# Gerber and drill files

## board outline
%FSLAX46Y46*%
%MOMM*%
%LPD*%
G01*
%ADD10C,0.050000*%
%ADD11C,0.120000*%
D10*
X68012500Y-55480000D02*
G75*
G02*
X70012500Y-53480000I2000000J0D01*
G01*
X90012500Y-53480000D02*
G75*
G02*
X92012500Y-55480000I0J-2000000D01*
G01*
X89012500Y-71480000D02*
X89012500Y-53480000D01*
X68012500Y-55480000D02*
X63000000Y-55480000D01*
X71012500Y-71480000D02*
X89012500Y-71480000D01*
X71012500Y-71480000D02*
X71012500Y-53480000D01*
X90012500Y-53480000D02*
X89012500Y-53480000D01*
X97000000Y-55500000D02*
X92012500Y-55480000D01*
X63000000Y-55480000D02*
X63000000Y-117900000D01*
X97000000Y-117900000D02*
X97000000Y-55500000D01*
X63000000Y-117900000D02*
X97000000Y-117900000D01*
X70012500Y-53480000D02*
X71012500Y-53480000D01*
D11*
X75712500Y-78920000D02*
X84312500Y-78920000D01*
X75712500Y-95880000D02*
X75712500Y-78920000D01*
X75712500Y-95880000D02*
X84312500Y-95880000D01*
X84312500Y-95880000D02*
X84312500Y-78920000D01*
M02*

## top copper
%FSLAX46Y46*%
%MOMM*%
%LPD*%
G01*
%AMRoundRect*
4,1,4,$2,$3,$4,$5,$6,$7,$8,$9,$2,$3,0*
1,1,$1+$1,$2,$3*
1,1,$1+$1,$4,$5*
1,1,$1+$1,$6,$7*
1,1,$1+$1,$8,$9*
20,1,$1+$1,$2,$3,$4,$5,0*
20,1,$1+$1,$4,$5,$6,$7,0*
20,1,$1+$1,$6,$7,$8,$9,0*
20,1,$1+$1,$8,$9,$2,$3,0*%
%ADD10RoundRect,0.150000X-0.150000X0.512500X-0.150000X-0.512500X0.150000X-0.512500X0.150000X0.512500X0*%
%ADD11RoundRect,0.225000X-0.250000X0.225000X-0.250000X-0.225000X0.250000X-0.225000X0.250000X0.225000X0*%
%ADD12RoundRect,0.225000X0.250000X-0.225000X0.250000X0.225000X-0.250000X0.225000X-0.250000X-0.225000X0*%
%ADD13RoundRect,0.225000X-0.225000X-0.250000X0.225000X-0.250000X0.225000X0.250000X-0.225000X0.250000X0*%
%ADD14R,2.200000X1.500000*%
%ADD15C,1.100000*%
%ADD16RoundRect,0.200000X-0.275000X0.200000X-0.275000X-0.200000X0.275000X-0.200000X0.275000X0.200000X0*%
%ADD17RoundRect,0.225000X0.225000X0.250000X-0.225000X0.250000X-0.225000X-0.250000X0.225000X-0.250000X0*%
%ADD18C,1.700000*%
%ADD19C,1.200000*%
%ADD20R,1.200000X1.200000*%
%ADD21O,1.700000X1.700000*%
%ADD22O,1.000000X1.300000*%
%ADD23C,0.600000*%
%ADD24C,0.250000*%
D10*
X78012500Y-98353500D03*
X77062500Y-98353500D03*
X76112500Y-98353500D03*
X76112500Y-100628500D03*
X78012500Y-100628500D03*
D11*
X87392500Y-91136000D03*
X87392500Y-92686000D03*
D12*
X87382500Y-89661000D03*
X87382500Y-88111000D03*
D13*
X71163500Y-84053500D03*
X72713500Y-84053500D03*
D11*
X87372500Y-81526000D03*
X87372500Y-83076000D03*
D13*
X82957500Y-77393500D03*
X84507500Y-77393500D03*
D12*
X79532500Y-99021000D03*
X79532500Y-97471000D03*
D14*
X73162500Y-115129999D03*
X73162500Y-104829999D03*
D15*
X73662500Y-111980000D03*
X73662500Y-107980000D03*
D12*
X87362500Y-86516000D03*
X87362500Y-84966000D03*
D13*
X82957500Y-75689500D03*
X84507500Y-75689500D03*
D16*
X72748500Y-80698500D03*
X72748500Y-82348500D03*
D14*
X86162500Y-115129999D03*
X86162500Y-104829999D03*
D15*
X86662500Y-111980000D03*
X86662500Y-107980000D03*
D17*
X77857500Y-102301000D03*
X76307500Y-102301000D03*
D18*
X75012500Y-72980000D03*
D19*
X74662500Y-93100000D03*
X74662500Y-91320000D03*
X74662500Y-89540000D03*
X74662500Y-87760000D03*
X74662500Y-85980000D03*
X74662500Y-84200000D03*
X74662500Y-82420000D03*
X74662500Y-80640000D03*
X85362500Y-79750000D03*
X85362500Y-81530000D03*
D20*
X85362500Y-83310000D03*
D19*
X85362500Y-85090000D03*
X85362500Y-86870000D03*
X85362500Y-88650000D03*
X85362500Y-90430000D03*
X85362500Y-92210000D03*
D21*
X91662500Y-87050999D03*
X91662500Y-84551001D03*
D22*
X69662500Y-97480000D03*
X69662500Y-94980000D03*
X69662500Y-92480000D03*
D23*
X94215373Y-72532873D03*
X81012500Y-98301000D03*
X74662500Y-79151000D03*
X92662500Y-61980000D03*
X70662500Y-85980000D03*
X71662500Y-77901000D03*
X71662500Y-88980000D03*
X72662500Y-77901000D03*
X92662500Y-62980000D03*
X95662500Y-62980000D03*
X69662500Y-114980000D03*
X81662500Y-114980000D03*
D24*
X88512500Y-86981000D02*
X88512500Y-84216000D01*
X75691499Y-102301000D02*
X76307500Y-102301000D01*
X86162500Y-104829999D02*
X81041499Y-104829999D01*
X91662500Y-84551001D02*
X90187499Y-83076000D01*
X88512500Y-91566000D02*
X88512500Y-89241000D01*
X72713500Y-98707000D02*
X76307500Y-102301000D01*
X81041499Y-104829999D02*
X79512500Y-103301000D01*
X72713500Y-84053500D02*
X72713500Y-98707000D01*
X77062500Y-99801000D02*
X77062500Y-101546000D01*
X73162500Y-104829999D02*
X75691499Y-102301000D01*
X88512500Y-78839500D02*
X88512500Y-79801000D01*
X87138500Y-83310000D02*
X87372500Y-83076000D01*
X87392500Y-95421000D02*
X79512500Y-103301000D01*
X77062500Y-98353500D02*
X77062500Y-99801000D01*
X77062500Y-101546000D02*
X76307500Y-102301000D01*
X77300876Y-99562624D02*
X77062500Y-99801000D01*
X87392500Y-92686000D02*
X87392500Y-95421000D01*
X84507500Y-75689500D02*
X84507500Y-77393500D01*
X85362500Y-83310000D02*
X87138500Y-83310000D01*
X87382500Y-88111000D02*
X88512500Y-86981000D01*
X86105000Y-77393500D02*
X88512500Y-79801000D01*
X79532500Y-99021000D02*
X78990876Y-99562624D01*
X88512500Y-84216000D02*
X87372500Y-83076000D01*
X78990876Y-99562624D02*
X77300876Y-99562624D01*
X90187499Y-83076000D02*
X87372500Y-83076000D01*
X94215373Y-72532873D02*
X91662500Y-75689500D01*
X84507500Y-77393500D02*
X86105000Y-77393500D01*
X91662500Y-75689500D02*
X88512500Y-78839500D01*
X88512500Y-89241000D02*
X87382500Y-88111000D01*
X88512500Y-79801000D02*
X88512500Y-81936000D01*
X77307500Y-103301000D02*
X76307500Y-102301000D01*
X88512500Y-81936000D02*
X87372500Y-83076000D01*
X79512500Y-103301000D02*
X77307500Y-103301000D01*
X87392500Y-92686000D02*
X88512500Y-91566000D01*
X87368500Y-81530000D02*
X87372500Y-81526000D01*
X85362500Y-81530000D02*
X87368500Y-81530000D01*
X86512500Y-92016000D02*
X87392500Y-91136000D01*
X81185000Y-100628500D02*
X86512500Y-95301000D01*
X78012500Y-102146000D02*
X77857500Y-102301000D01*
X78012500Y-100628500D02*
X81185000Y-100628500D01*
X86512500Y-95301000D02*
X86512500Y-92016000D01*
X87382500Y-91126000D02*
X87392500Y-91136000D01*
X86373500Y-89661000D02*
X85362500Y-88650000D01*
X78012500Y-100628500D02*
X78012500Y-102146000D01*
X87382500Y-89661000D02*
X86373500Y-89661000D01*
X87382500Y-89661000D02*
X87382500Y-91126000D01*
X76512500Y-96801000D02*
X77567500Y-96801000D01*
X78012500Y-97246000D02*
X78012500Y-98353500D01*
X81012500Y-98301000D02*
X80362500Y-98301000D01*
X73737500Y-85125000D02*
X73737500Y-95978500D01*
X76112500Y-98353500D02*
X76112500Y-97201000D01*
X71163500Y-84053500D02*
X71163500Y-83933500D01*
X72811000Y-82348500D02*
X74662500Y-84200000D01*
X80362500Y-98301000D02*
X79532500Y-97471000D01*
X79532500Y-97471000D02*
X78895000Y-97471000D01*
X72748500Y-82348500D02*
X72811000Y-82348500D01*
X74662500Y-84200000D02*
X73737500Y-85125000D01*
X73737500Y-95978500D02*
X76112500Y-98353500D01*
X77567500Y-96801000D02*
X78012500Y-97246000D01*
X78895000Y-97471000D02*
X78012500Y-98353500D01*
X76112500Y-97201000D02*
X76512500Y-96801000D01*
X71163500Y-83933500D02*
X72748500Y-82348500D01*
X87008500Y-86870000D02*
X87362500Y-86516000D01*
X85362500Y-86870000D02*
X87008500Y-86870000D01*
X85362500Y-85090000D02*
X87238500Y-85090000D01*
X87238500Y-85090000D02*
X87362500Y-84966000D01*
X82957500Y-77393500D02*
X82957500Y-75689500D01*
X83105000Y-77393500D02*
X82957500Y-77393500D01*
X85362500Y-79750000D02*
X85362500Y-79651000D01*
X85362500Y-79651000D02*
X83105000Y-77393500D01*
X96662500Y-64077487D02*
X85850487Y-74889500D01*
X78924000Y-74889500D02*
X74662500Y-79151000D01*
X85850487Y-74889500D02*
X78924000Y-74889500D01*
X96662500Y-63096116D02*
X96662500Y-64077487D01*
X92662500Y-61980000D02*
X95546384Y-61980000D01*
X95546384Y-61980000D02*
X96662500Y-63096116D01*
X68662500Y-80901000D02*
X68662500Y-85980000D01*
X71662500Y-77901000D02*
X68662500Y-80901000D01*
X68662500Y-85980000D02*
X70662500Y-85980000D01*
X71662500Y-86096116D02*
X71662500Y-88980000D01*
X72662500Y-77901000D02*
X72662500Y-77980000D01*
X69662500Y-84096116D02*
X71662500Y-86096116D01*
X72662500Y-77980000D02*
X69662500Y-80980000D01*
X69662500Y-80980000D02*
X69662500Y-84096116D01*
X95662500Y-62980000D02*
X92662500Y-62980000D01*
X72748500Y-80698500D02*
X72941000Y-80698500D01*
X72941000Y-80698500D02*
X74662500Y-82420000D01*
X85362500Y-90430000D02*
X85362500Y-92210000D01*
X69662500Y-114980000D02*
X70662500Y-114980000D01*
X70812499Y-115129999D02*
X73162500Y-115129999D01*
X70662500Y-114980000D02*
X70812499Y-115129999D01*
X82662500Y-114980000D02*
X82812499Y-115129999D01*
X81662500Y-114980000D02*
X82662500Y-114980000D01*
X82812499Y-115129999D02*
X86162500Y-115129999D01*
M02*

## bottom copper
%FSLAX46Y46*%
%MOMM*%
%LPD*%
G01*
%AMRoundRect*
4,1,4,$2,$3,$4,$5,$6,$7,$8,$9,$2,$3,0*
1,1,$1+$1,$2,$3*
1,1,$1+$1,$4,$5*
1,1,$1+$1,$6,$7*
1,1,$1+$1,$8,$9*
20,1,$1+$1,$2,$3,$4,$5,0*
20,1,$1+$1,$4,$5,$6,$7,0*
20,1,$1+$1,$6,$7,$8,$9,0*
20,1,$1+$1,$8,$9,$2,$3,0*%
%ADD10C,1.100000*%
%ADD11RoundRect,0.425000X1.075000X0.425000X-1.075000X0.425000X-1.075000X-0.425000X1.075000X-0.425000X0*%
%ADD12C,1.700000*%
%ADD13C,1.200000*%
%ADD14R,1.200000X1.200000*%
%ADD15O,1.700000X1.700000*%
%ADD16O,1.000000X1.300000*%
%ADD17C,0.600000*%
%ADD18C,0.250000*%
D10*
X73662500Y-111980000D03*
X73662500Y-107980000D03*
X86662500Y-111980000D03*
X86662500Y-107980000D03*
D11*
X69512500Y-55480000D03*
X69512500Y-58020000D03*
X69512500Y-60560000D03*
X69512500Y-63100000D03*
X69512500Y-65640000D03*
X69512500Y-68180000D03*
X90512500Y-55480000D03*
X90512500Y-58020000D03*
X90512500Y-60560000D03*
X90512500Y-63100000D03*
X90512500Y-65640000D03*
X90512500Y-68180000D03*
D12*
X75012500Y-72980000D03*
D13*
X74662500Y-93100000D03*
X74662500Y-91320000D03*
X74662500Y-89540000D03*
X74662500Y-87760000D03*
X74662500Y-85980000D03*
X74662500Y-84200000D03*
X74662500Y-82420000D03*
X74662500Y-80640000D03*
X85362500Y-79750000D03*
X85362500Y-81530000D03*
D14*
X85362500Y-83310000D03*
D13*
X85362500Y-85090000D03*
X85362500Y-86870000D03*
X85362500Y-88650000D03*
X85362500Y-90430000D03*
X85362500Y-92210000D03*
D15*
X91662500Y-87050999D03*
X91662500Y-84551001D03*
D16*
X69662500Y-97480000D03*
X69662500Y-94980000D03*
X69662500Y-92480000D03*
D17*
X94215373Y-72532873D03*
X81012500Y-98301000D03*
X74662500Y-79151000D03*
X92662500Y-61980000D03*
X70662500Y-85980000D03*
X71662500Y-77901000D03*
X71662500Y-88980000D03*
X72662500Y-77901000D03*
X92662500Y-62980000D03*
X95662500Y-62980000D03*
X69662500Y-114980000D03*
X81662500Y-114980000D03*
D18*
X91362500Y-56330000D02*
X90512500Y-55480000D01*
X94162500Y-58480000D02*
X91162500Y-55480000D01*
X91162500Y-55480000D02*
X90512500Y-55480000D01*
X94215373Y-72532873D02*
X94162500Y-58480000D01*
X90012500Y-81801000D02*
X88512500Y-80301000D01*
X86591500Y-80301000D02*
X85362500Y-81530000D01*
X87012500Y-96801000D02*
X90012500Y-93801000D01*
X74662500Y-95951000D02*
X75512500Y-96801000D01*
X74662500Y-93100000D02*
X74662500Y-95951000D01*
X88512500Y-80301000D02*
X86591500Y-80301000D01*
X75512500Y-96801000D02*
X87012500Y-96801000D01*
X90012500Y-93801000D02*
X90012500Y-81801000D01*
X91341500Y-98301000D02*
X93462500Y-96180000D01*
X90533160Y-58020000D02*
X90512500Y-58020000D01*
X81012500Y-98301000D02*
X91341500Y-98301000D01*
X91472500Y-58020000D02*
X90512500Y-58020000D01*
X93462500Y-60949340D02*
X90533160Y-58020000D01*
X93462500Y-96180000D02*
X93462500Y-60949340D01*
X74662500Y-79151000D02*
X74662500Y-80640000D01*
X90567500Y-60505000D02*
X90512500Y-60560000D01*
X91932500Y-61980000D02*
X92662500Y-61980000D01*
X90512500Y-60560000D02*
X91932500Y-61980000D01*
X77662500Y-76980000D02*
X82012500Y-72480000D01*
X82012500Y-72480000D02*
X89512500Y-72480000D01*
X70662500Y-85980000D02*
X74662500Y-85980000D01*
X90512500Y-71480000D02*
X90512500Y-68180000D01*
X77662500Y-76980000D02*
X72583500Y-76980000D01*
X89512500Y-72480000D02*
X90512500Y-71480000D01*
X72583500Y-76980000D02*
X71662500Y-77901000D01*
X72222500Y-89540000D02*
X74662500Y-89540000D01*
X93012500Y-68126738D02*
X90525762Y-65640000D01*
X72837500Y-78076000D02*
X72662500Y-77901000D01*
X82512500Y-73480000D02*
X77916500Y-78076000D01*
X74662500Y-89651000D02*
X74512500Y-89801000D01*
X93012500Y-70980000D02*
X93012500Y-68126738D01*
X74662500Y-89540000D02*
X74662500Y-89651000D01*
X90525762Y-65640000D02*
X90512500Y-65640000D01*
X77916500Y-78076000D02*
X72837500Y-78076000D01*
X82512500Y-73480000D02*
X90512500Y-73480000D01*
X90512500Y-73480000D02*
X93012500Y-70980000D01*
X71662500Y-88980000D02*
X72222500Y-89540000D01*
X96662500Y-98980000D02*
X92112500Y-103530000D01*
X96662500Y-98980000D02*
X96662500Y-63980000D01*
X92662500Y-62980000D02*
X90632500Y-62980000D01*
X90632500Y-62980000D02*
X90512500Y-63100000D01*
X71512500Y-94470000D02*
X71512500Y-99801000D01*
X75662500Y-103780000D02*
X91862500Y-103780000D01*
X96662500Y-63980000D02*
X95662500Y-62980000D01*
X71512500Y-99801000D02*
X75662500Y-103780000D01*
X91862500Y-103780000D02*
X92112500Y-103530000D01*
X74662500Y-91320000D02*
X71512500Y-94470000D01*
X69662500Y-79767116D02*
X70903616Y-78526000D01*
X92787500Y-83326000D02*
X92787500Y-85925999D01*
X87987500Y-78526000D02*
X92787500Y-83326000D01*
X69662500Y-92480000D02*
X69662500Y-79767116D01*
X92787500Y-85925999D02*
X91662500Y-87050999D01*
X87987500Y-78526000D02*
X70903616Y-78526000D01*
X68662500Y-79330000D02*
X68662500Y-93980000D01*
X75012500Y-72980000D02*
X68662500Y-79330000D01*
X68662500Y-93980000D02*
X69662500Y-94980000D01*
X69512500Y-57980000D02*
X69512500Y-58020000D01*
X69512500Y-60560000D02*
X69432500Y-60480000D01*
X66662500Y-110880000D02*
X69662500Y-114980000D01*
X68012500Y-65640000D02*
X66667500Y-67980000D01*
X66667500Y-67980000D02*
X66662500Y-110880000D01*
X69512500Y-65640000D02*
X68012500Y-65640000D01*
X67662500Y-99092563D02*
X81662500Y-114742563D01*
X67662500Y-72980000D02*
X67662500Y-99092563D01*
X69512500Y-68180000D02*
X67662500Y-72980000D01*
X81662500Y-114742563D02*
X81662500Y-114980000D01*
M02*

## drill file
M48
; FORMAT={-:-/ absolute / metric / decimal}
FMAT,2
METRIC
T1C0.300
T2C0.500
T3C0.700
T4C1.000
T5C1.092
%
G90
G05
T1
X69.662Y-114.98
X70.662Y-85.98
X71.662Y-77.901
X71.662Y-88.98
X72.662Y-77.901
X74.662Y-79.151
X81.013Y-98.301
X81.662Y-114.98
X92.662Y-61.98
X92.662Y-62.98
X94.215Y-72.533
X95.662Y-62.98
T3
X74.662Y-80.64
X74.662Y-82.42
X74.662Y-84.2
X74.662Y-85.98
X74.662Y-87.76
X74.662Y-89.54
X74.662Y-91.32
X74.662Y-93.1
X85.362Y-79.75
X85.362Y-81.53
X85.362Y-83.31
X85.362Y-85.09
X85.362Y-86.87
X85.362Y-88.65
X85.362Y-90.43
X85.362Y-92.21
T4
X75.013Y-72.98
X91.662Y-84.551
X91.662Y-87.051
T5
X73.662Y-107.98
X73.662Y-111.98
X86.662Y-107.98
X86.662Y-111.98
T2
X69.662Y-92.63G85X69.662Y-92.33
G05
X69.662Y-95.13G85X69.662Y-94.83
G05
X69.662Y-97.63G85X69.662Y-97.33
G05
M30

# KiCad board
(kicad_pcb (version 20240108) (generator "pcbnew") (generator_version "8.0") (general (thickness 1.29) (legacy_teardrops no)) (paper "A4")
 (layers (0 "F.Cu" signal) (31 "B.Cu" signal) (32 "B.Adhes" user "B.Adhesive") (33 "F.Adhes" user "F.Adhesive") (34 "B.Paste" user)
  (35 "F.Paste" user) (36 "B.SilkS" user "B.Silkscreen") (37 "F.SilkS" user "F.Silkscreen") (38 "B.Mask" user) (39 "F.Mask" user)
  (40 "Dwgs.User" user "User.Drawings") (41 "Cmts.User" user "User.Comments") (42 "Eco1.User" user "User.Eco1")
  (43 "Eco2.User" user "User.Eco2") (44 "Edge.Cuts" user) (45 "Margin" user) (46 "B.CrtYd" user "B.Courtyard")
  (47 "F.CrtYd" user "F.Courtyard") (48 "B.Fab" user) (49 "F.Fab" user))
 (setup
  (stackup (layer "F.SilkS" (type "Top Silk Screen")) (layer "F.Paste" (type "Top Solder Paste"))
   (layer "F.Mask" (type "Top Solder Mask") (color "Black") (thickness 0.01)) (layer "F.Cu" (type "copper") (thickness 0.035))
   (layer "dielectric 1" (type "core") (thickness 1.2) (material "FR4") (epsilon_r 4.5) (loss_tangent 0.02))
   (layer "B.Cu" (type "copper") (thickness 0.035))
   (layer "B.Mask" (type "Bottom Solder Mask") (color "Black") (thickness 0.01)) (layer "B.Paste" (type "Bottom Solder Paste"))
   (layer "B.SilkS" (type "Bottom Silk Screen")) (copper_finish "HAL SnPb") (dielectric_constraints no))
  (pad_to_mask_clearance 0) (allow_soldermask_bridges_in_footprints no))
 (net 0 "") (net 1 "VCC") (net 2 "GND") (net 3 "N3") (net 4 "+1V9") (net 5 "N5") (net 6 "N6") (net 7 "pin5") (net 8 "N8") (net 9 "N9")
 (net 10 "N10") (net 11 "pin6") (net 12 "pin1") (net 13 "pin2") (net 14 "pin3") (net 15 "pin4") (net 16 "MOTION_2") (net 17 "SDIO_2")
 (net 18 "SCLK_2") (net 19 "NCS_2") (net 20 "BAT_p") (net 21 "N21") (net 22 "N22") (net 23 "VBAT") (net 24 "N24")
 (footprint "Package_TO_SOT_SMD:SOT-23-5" (layer "F.Cu") (at 77.0625 99.491 -90)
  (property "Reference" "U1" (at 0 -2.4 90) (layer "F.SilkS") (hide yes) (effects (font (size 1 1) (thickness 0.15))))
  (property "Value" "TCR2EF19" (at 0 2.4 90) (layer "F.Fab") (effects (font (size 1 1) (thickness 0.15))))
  (pad "1" smd roundrect (at -1.1375 -0.95 270) (size 1.325 0.6) (layers "F.Cu" "F.Paste" "F.Mask") (roundrect_rratio 0.25) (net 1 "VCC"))
  (pad "2" smd roundrect (at -1.1375 0 270) (size 1.325 0.6) (layers "F.Cu" "F.Paste" "F.Mask") (roundrect_rratio 0.25) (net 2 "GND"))
  (pad "3" smd roundrect (at -1.1375 0.95 270) (size 1.325 0.6) (layers "F.Cu" "F.Paste" "F.Mask") (roundrect_rratio 0.25) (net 1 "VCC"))
  (pad "4" smd roundrect (at 1.1375 0.95 270) (size 1.325 0.6) (layers "F.Cu" "F.Paste" "F.Mask") (roundrect_rratio 0.25) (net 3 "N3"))
  (pad "5" smd roundrect (at 1.1375 -0.95 270) (size 1.325 0.6) (layers "F.Cu" "F.Paste" "F.Mask") (roundrect_rratio 0.25) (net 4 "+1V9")))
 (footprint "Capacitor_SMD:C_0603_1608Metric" (layer "F.Cu") (at 87.3925 91.911 -90)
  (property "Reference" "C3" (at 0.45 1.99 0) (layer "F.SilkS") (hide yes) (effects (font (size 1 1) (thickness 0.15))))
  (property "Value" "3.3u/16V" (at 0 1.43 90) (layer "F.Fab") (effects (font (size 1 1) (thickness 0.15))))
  (pad "1" smd roundrect (at -0.775 0 270) (size 0.9 0.95) (layers "F.Cu" "F.Paste" "F.Mask") (roundrect_rratio 0.25) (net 4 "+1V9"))
  (pad "2" smd roundrect (at 0.775 0 270) (size 0.9 0.95) (layers "F.Cu" "F.Paste" "F.Mask") (roundrect_rratio 0.25) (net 2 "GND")))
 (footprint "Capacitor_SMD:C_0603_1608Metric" (layer "F.Cu") (at 87.3825 88.886 90)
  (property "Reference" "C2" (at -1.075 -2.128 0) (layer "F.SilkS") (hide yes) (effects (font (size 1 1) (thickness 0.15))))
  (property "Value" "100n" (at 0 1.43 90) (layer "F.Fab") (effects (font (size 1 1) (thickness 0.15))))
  (pad "1" smd roundrect (at -0.775 0 90) (size 0.9 0.95) (layers "F.Cu" "F.Paste" "F.Mask") (roundrect_rratio 0.25) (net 4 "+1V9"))
  (pad "2" smd roundrect (at 0.775 0 90) (size 0.9 0.95) (layers "F.Cu" "F.Paste" "F.Mask") (roundrect_rratio 0.25) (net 2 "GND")))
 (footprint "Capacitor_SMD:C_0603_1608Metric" (layer "F.Cu") (at 71.9385 84.0535)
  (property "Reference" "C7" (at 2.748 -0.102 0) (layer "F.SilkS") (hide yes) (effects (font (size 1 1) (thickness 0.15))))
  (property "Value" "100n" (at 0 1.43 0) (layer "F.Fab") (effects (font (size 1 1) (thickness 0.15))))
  (pad "1" smd roundrect (at -0.775 0) (size 0.9 0.95) (layers "F.Cu" "F.Paste" "F.Mask") (roundrect_rratio 0.25) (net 1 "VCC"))
  (pad "2" smd roundrect (at 0.775 0) (size 0.9 0.95) (layers "F.Cu" "F.Paste" "F.Mask") (roundrect_rratio 0.25) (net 2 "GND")))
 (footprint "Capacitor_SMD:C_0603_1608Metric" (layer "F.Cu") (at 87.3725 82.301 -90)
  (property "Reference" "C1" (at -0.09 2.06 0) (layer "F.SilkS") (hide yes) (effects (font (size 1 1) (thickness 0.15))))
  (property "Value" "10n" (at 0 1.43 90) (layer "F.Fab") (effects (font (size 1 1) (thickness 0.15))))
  (pad "1" smd roundrect (at -0.775 0 270) (size 0.9 0.95) (layers "F.Cu" "F.Paste" "F.Mask") (roundrect_rratio 0.25) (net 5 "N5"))
  (pad "2" smd roundrect (at 0.775 0 270) (size 0.9 0.95) (layers "F.Cu" "F.Paste" "F.Mask") (roundrect_rratio 0.25) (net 2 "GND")))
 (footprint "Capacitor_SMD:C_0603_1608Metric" (layer "F.Cu") (at 83.7325 77.3935)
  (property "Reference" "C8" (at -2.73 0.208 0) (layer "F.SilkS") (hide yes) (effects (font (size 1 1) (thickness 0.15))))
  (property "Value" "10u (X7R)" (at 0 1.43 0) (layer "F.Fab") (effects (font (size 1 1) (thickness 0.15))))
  (pad "1" smd roundrect (at -0.775 0) (size 0.9 0.95) (layers "F.Cu" "F.Paste" "F.Mask") (roundrect_rratio 0.25) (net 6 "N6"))
  (pad "2" smd roundrect (at 0.775 0) (size 0.9 0.95) (layers "F.Cu" "F.Paste" "F.Mask") (roundrect_rratio 0.25) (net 2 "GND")))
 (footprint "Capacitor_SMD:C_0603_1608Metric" (layer "F.Cu") (at 79.5325 98.246 90)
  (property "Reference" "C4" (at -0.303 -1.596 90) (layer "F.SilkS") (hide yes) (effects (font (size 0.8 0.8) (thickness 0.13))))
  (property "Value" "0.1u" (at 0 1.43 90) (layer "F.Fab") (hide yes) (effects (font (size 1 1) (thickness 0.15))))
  (pad "1" smd roundrect (at -0.775 0 90) (size 0.9 0.95) (layers "F.Cu" "F.Paste" "F.Mask") (roundrect_rratio 0.25) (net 2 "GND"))
  (pad "2" smd roundrect (at 0.775 0 90) (size 0.9 0.95) (layers "F.Cu" "F.Paste" "F.Mask") (roundrect_rratio 0.25) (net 1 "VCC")))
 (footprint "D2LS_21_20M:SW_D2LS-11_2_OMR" (layer "F.Cu") (at 73.6625 109.98 90)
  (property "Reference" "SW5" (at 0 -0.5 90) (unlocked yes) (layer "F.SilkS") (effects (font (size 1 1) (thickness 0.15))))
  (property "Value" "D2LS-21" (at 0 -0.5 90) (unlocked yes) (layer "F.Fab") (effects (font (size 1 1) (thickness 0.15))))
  (pad "1" smd rect (at -5.149999 -0.5 90) (size 1.5 2.2) (layers "F.Cu" "F.Paste" "F.Mask") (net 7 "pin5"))
  (pad "2" smd rect (at 5.150001 -0.5 90) (size 1.5 2.2) (layers "F.Cu" "F.Paste" "F.Mask") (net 2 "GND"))
  (pad "3" thru_hole circle (at -2 0 90) (size 1.1 1.1) (drill 1.0922) (layers "*.Cu" "*.Mask") (remove_unused_layers no))
  (pad "4" thru_hole circle (at 2 0 90) (size 1.1 1.1) (drill 1.0922) (layers "*.Cu" "*.Mask") (remove_unused_layers no)))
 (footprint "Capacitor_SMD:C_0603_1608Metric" (layer "F.Cu") (at 87.3625 85.741 90)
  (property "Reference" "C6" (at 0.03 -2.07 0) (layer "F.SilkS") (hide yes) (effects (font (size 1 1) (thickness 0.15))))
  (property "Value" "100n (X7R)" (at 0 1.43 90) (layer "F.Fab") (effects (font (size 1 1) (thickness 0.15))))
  (pad "1" smd roundrect (at -0.775 0 90) (size 0.9 0.95) (layers "F.Cu" "F.Paste" "F.Mask") (roundrect_rratio 0.25) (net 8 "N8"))
  (pad "2" smd roundrect (at 0.775 0 90) (size 0.9 0.95) (layers "F.Cu" "F.Paste" "F.Mask") (roundrect_rratio 0.25) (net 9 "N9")))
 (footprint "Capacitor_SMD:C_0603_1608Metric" (layer "F.Cu") (at 83.7325 75.6895)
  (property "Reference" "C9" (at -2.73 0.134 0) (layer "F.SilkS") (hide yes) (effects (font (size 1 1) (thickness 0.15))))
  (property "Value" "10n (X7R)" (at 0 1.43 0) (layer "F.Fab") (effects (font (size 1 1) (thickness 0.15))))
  (pad "1" smd roundrect (at -0.775 0) (size 0.9 0.95) (layers "F.Cu" "F.Paste" "F.Mask") (roundrect_rratio 0.25) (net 6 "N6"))
  (pad "2" smd roundrect (at 0.775 0) (size 0.9 0.95) (layers "F.Cu" "F.Paste" "F.Mask") (roundrect_rratio 0.25) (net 2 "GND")))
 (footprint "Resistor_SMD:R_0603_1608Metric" (layer "F.Cu") (at 72.7485 81.5235 -90)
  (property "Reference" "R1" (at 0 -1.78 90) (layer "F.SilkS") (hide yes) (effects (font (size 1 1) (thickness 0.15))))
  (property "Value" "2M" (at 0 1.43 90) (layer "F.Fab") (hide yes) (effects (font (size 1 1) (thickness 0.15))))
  (pad "1" smd roundrect (at -0.825 0 270) (size 0.8 0.95) (layers "F.Cu" "F.Paste" "F.Mask") (roundrect_rratio 0.25) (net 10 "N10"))
  (pad "2" smd roundrect (at 0.825 0 270) (size 0.8 0.95) (layers "F.Cu" "F.Paste" "F.Mask") (roundrect_rratio 0.25) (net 1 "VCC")))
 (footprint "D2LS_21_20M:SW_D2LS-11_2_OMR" (layer "F.Cu") (at 86.6625 109.98 90)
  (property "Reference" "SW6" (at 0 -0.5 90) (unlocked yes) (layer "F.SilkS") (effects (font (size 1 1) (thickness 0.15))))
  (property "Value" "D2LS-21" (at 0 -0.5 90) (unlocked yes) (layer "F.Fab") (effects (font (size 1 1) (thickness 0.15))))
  (pad "1" smd rect (at -5.149999 -0.5 90) (size 1.5 2.2) (layers "F.Cu" "F.Paste" "F.Mask") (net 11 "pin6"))
  (pad "2" smd rect (at 5.150001 -0.5 90) (size 1.5 2.2) (layers "F.Cu" "F.Paste" "F.Mask") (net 2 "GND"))
  (pad "3" thru_hole circle (at -2 0 90) (size 1.1 1.1) (drill 1.0922) (layers "*.Cu" "*.Mask") (remove_unused_layers no))
  (pad "4" thru_hole circle (at 2 0 90) (size 1.1 1.1) (drill 1.0922) (layers "*.Cu" "*.Mask") (remove_unused_layers no)))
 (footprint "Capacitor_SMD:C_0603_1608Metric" (layer "F.Cu") (at 77.0825 102.301 180)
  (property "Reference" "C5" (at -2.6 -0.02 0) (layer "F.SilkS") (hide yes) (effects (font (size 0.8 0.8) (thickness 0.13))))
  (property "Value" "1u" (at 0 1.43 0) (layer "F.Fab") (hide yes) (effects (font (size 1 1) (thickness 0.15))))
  (pad "1" smd roundrect (at -0.775 0 180) (size 0.9 0.95) (layers "F.Cu" "F.Paste" "F.Mask") (roundrect_rratio 0.25) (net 4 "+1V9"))
  (pad "2" smd roundrect (at 0.775 0 180) (size 0.9 0.95) (layers "F.Cu" "F.Paste" "F.Mask") (roundrect_rratio 0.25) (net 2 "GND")))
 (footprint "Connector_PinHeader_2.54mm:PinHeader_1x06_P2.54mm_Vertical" (layer "B.Cu") (at 69.5125 55.48 180)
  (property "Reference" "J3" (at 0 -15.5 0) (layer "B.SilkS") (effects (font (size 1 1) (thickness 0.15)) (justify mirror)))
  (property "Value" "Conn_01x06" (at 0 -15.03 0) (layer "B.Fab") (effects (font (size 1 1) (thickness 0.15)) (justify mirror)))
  (pad "1" smd roundrect (at 0 0 180) (size 3 1.7) (layers "B.Cu" "B.Paste" "B.Mask") (roundrect_rratio 0.25) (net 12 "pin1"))
  (pad "2" smd roundrect (at 0 -2.54 180) (size 3 1.7) (layers "B.Cu" "B.Paste" "B.Mask") (roundrect_rratio 0.25) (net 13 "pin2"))
  (pad "3" smd roundrect (at 0 -5.08 180) (size 3 1.7) (layers "B.Cu" "B.Paste" "B.Mask") (roundrect_rratio 0.25) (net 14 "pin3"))
  (pad "4" smd roundrect (at 0 -7.62 180) (size 3 1.7) (layers "B.Cu" "B.Paste" "B.Mask") (roundrect_rratio 0.25) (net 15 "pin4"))
  (pad "5" smd roundrect (at 0 -10.16 180) (size 3 1.7) (layers "B.Cu" "B.Paste" "B.Mask") (roundrect_rratio 0.25) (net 7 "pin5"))
  (pad "6" smd roundrect (at 0 -12.7 180) (size 3 1.7) (layers "B.Cu" "B.Paste" "B.Mask") (roundrect_rratio 0.25) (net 11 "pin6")))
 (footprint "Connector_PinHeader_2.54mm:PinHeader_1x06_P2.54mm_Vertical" (layer "B.Cu") (at 90.5125 55.48 180)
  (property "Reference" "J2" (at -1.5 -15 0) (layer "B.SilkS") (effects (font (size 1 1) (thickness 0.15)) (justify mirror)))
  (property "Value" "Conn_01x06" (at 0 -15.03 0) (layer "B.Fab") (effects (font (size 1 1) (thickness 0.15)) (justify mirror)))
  (pad "1" smd roundrect (at 0 0 180) (size 3 1.7) (layers "B.Cu" "B.Paste" "B.Mask") (roundrect_rratio 0.25) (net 2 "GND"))
  (pad "2" smd roundrect (at 0 -2.54 180) (size 3 1.7) (layers "B.Cu" "B.Paste" "B.Mask") (roundrect_rratio 0.25) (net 1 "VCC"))
  (pad "3" smd roundrect (at 0 -5.08 180) (size 3 1.7) (layers "B.Cu" "B.Paste" "B.Mask") (roundrect_rratio 0.25) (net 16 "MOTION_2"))
  (pad "4" smd roundrect (at 0 -7.62 180) (size 3 1.7) (layers "B.Cu" "B.Paste" "B.Mask") (roundrect_rratio 0.25) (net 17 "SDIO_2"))
  (pad "5" smd roundrect (at 0 -10.16 180) (size 3 1.7) (layers "B.Cu" "B.Paste" "B.Mask") (roundrect_rratio 0.25) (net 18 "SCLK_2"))
  (pad "6" smd roundrect (at 0 -12.7 180) (size 3 1.7) (layers "B.Cu" "B.Paste" "B.Mask") (roundrect_rratio 0.25) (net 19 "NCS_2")))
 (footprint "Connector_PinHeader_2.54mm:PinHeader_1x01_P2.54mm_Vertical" (layer "B.Cu") (at 75.0125 72.98 180)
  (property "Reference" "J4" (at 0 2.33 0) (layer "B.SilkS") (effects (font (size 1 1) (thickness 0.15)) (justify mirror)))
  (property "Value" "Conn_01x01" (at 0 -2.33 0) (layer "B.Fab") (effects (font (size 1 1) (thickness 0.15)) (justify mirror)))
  (pad "1" thru_hole circle (at 0 0 180) (size 1.7 1.7) (drill 1) (layers "*.Cu" "*.Mask") (remove_unused_layers no) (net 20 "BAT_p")))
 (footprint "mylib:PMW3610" (layer "B.Cu") (at 74.6625 93.1)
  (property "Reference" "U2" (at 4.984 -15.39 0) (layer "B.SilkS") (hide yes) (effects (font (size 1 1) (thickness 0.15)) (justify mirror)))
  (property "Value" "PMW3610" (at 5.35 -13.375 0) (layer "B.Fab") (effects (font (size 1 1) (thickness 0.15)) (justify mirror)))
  (fp_line (start 1.05 -14.18) (end 9.65 -14.18) (stroke (width 0.12) (type solid)) (layer "Edge.Cuts"))
  (fp_line (start 1.05 2.78) (end 1.05 -14.18) (stroke (width 0.12) (type solid)) (layer "Edge.Cuts"))
  (fp_line (start 1.05 2.78) (end 9.65 2.78) (stroke (width 0.12) (type solid)) (layer "Edge.Cuts"))
  (fp_line (start 9.65 2.78) (end 9.65 -14.18) (stroke (width 0.12) (type solid)) (layer "Edge.Cuts"))
  (pad "1" thru_hole circle (at 0 0) (size 1.2 1.2) (drill 0.7) (layers "*.Cu" "*.Mask") (remove_unused_layers no) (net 5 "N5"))
  (pad "2" thru_hole circle (at 0 -1.78) (size 1.2 1.2) (drill 0.7) (layers "*.Cu" "*.Mask") (remove_unused_layers no) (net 17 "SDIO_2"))
  (pad "3" thru_hole circle (at 0 -3.56) (size 1.2 1.2) (drill 0.7) (layers "*.Cu" "*.Mask") (remove_unused_layers no) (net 18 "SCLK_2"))
  (pad "4" thru_hole circle (at 0 -5.34) (size 1.2 1.2) (drill 0.7) (layers "*.Cu" "*.Mask") (remove_unused_layers no) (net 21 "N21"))
  (pad "5" thru_hole circle (at 0 -7.12) (size 1.2 1.2) (drill 0.7) (layers "*.Cu" "*.Mask") (remove_unused_layers no) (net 19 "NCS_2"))
  (pad "6" thru_hole circle (at 0 -8.9) (size 1.2 1.2) (drill 0.7) (layers "*.Cu" "*.Mask") (remove_unused_layers no) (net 1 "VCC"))
  (pad "7" thru_hole circle (at 0 -10.68) (size 1.2 1.2) (drill 0.7) (layers "*.Cu" "*.Mask") (remove_unused_layers no) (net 10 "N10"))
  (pad "8" thru_hole circle (at 0 -12.46) (size 1.2 1.2) (drill 0.7) (layers "*.Cu" "*.Mask") (remove_unused_layers no) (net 16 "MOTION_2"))
  (pad "9" thru_hole circle (at 10.7 -13.35) (size 1.2 1.2) (drill 0.7) (layers "*.Cu" "*.Mask") (remove_unused_layers no) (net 6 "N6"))
  (pad "10" thru_hole circle (at 10.7 -11.57) (size 1.2 1.2) (drill 0.7) (layers "*.Cu" "*.Mask") (remove_unused_layers no) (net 5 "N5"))
  (pad "11" thru_hole rect (at 10.7 -9.79) (size 1.2 1.2) (drill 0.7) (layers "*.Cu" "*.Mask") (remove_unused_layers no) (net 2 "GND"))
  (pad "12" thru_hole circle (at 10.7 -8.01) (size 1.2 1.2) (drill 0.7) (layers "*.Cu" "*.Mask") (remove_unused_layers no) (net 9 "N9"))
  (pad "13" thru_hole circle (at 10.7 -6.23) (size 1.2 1.2) (drill 0.7) (layers "*.Cu" "*.Mask") (remove_unused_layers no) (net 8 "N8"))
  (pad "14" thru_hole circle (at 10.7 -4.45) (size 1.2 1.2) (drill 0.7) (layers "*.Cu" "*.Mask") (remove_unused_layers no) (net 4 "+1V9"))
  (pad "15" thru_hole circle (at 10.7 -2.67) (size 1.2 1.2) (drill 0.7) (layers "*.Cu" "*.Mask") (remove_unused_layers no) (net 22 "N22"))
  (pad "16" thru_hole circle (at 10.7 -0.89) (size 1.2 1.2) (drill 0.7) (layers "*.Cu" "*.Mask") (remove_unused_layers no) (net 22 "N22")))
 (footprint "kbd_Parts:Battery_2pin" (layer "B.Cu") (at 91.6625 85.801 90)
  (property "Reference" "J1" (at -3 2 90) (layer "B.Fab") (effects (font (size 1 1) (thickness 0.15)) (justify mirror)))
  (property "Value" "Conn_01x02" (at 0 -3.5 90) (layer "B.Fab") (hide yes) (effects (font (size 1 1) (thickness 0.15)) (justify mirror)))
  (pad "1" thru_hole oval (at -1.249999 0 90) (size 1.7 1.7) (drill oval 1) (layers "*.Cu" "*.Mask") (remove_unused_layers no)
   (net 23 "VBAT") (clearance 0.15))
  (pad "2" thru_hole oval (at 1.249999 0 90) (size 1.7 1.7) (drill oval 1) (layers "*.Cu" "*.Mask") (remove_unused_layers no) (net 2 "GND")
   (clearance 0.15)))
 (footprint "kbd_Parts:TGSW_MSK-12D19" (layer "B.Cu") (at 70.7125 94.98 90)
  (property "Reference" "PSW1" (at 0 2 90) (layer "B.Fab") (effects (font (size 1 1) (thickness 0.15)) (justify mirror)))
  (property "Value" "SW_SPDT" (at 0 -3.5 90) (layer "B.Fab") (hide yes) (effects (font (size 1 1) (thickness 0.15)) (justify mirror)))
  (pad "1" thru_hole oval (at -2.5 -1.05 90) (size 1.3 1) (drill oval 0.8 0.5) (layers "*.Cu" "*.Mask") (remove_unused_layers no)
   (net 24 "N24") (clearance 0.15))
  (pad "2" thru_hole oval (at 0 -1.05 90) (size 1.3 1) (drill oval 0.8 0.5) (layers "*.Cu" "*.Mask") (remove_unused_layers no)
   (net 20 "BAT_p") (clearance 0.15))
  (pad "3" thru_hole oval (at 2.5 -1.05 90) (size 1.3 1) (drill oval 0.8 0.5) (layers "*.Cu" "*.Mask") (remove_unused_layers no)
   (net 23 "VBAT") (clearance 0.15)))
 (gr_arc (start 68.0125 55.48) (mid 68.598286 54.065786) (end 70.0125 53.48) (stroke (width 0.05) (type default)) (layer "Edge.Cuts"))
 (gr_arc (start 90.0125 53.48) (mid 91.426714 54.065786) (end 92.0125 55.48) (stroke (width 0.05) (type default)) (layer "Edge.Cuts"))
 (gr_line (start 89.0125 71.48) (end 89.0125 53.48) (stroke (width 0.05) (type default)) (layer "Edge.Cuts"))
 (gr_line (start 68.0125 55.48) (end 63 55.48) (stroke (width 0.05) (type default)) (layer "Edge.Cuts"))
 (gr_line (start 71.0125 71.48) (end 89.0125 71.48) (stroke (width 0.05) (type default)) (layer "Edge.Cuts"))
 (gr_line (start 71.0125 71.48) (end 71.0125 53.48) (stroke (width 0.05) (type default)) (layer "Edge.Cuts"))
 (gr_line (start 90.0125 53.48) (end 89.0125 53.48) (stroke (width 0.05) (type default)) (layer "Edge.Cuts"))
 (gr_line (start 97 55.5) (end 92.0125 55.48) (stroke (width 0.05) (type default)) (layer "Edge.Cuts"))
 (gr_line (start 63 55.48) (end 63 117.9) (stroke (width 0.05) (type default)) (layer "Edge.Cuts"))
 (gr_line (start 97 117.9) (end 97 55.5) (stroke (width 0.05) (type default)) (layer "Edge.Cuts"))
 (gr_line (start 63 117.9) (end 97 117.9) (stroke (width 0.05) (type default)) (layer "Edge.Cuts"))
 (gr_line (start 70.0125 53.48) (end 71.0125 53.48) (stroke (width 0.05) (type default)) (layer "Edge.Cuts"))
 (segment (start 88.5125 86.981) (end 88.5125 84.216) (width 0.25) (layer "F.Cu") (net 2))
 (segment (start 75.691499 102.301) (end 76.3075 102.301) (width 0.25) (layer "F.Cu") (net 2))
 (segment (start 86.1625 104.829999) (end 81.041499 104.829999) (width 0.25) (layer "F.Cu") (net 2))
 (segment (start 91.6625 84.551001) (end 90.187499 83.076) (width 0.25) (layer "F.Cu") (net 2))
 (segment (start 88.5125 91.566) (end 88.5125 89.241) (width 0.25) (layer "F.Cu") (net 2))
 (segment (start 72.7135 98.707) (end 76.3075 102.301) (width 0.25) (layer "F.Cu") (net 2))
 (segment (start 81.041499 104.829999) (end 79.5125 103.301) (width 0.25) (layer "F.Cu") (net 2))
 (segment (start 72.7135 84.0535) (end 72.7135 98.707) (width 0.25) (layer "F.Cu") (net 2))
 (segment (start 77.0625 99.801) (end 77.0625 101.546) (width 0.25) (layer "F.Cu") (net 2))
 (segment (start 73.1625 104.829999) (end 75.691499 102.301) (width 0.25) (layer "F.Cu") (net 2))
 (segment (start 88.5125 78.8395) (end 88.5125 79.801) (width 0.25) (layer "F.Cu") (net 2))
 (segment (start 87.1385 83.31) (end 87.3725 83.076) (width 0.25) (layer "F.Cu") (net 2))
 (segment (start 87.3925 95.421) (end 79.5125 103.301) (width 0.25) (layer "F.Cu") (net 2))
 (segment (start 77.0625 98.3535) (end 77.0625 99.801) (width 0.25) (layer "F.Cu") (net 2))
 (segment (start 77.0625 101.546) (end 76.3075 102.301) (width 0.25) (layer "F.Cu") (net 2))
 (segment (start 77.300876 99.562624) (end 77.0625 99.801) (width 0.25) (layer "F.Cu") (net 2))
 (segment (start 87.3925 92.686) (end 87.3925 95.421) (width 0.25) (layer "F.Cu") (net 2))
 (segment (start 84.5075 75.6895) (end 84.5075 77.3935) (width 0.25) (layer "F.Cu") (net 2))
 (segment (start 85.3625 83.31) (end 87.1385 83.31) (width 0.25) (layer "F.Cu") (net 2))
 (segment (start 87.3825 88.111) (end 88.5125 86.981) (width 0.25) (layer "F.Cu") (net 2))
 (segment (start 86.105 77.3935) (end 88.5125 79.801) (width 0.25) (layer "F.Cu") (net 2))
 (segment (start 79.5325 99.021) (end 78.990876 99.562624) (width 0.25) (layer "F.Cu") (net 2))
 (segment (start 88.5125 84.216) (end 87.3725 83.076) (width 0.25) (layer "F.Cu") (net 2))
 (segment (start 78.990876 99.562624) (end 77.300876 99.562624) (width 0.25) (layer "F.Cu") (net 2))
 (segment (start 90.187499 83.076) (end 87.3725 83.076) (width 0.25) (layer "F.Cu") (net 2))
 (segment (start 94.215373 72.532873) (end 91.6625 75.6895) (width 0.25) (layer "F.Cu") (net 2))
 (segment (start 84.5075 77.3935) (end 86.105 77.3935) (width 0.25) (layer "F.Cu") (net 2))
 (segment (start 91.6625 75.6895) (end 88.5125 78.8395) (width 0.25) (layer "F.Cu") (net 2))
 (segment (start 88.5125 89.241) (end 87.3825 88.111) (width 0.25) (layer "F.Cu") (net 2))
 (segment (start 88.5125 79.801) (end 88.5125 81.936) (width 0.25) (layer "F.Cu") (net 2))
 (segment (start 77.3075 103.301) (end 76.3075 102.301) (width 0.25) (layer "F.Cu") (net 2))
 (segment (start 88.5125 81.936) (end 87.3725 83.076) (width 0.25) (layer "F.Cu") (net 2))
 (segment (start 79.5125 103.301) (end 77.3075 103.301) (width 0.25) (layer "F.Cu") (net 2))
 (segment (start 87.3925 92.686) (end 88.5125 91.566) (width 0.25) (layer "F.Cu") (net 2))
 (via (at 94.215373 72.532873) (size 0.6) (drill 0.3) (layers "F.Cu" "B.Cu") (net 2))
 (segment (start 91.3625 56.33) (end 90.5125 55.48) (width 0.25) (layer "B.Cu") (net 2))
 (segment (start 94.1625 58.48) (end 91.1625 55.48) (width 0.25) (layer "B.Cu") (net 2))
 (segment (start 91.1625 55.48) (end 90.5125 55.48) (width 0.25) (layer "B.Cu") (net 2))
 (segment (start 94.215373 72.532873) (end 94.1625 58.48) (width 0.25) (layer "B.Cu") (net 2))
 (segment (start 87.3685 81.53) (end 87.3725 81.526) (width 0.25) (layer "F.Cu") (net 5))
 (segment (start 85.3625 81.53) (end 87.3685 81.53) (width 0.25) (layer "F.Cu") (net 5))
 (segment (start 90.0125 81.801) (end 88.5125 80.301) (width 0.25) (layer "B.Cu") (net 5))
 (segment (start 86.5915 80.301) (end 85.3625 81.53) (width 0.25) (layer "B.Cu") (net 5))
 (segment (start 87.0125 96.801) (end 90.0125 93.801) (width 0.25) (layer "B.Cu") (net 5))
 (segment (start 74.6625 95.951) (end 75.5125 96.801) (width 0.25) (layer "B.Cu") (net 5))
 (segment (start 74.6625 93.1) (end 74.6625 95.951) (width 0.25) (layer "B.Cu") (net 5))
 (segment (start 88.5125 80.301) (end 86.5915 80.301) (width 0.25) (layer "B.Cu") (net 5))
 (segment (start 75.5125 96.801) (end 87.0125 96.801) (width 0.25) (layer "B.Cu") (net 5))
 (segment (start 90.0125 93.801) (end 90.0125 81.801) (width 0.25) (layer "B.Cu") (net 5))
 (segment (start 86.5125 92.016) (end 87.3925 91.136) (width 0.25) (layer "F.Cu") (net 4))
 (segment (start 81.185 100.6285) (end 86.5125 95.301) (width 0.25) (layer "F.Cu") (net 4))
 (segment (start 78.0125 102.146) (end 77.8575 102.301) (width 0.25) (layer "F.Cu") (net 4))
 (segment (start 78.0125 100.6285) (end 81.185 100.6285) (width 0.25) (layer "F.Cu") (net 4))
 (segment (start 86.5125 95.301) (end 86.5125 92.016) (width 0.25) (layer "F.Cu") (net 4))
 (segment (start 87.3825 91.126) (end 87.3925 91.136) (width 0.25) (layer "F.Cu") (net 4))
 (segment (start 86.3735 89.661) (end 85.3625 88.65) (width 0.25) (layer "F.Cu") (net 4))
 (segment (start 78.0125 100.6285) (end 78.0125 102.146) (width 0.25) (layer "F.Cu") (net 4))
 (segment (start 87.3825 89.661) (end 86.3735 89.661) (width 0.25) (layer "F.Cu") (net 4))
 (segment (start 87.3825 89.661) (end 87.3825 91.126) (width 0.25) (layer "F.Cu") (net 4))
 (segment (start 76.5125 96.801) (end 77.5675 96.801) (width 0.25) (layer "F.Cu") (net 1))
 (segment (start 78.0125 97.246) (end 78.0125 98.3535) (width 0.25) (layer "F.Cu") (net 1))
 (segment (start 81.0125 98.301) (end 80.3625 98.301) (width 0.25) (layer "F.Cu") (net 1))
 (segment (start 73.7375 85.125) (end 73.7375 95.9785) (width 0.25) (layer "F.Cu") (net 1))
 (segment (start 76.1125 98.3535) (end 76.1125 97.201) (width 0.25) (layer "F.Cu") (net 1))
 (segment (start 71.1635 84.0535) (end 71.1635 83.9335) (width 0.25) (layer "F.Cu") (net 1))
 (segment (start 72.811 82.3485) (end 74.6625 84.2) (width 0.25) (layer "F.Cu") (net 1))
 (segment (start 80.3625 98.301) (end 79.5325 97.471) (width 0.25) (layer "F.Cu") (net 1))
 (segment (start 79.5325 97.471) (end 78.895 97.471) (width 0.25) (layer "F.Cu") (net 1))
 (segment (start 72.7485 82.3485) (end 72.811 82.3485) (width 0.25) (layer "F.Cu") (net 1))
 (segment (start 74.6625 84.2) (end 73.7375 85.125) (width 0.25) (layer "F.Cu") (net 1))
 (segment (start 73.7375 95.9785) (end 76.1125 98.3535) (width 0.25) (layer "F.Cu") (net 1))
 (segment (start 77.5675 96.801) (end 78.0125 97.246) (width 0.25) (layer "F.Cu") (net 1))
 (segment (start 78.895 97.471) (end 78.0125 98.3535) (width 0.25) (layer "F.Cu") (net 1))
 (segment (start 76.1125 97.201) (end 76.5125 96.801) (width 0.25) (layer "F.Cu") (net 1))
 (segment (start 71.1635 83.9335) (end 72.7485 82.3485) (width 0.25) (layer "F.Cu") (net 1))
 (via (at 81.0125 98.301) (size 0.6) (drill 0.3) (layers "F.Cu" "B.Cu") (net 1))
 (segment (start 91.3415 98.301) (end 93.4625 96.18) (width 0.25) (layer "B.Cu") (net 1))
 (segment (start 90.53316 58.02) (end 90.5125 58.02) (width 0.25) (layer "B.Cu") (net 1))
 (segment (start 81.0125 98.301) (end 91.3415 98.301) (width 0.25) (layer "B.Cu") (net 1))
 (segment (start 91.4725 58.02) (end 90.5125 58.02) (width 0.25) (layer "B.Cu") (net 1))
 (segment (start 93.4625 60.94934) (end 90.53316 58.02) (width 0.25) (layer "B.Cu") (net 1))
 (segment (start 93.4625 96.18) (end 93.4625 60.94934) (width 0.25) (layer "B.Cu") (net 1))
 (segment (start 87.0085 86.87) (end 87.3625 86.516) (width 0.25) (layer "F.Cu") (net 8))
 (segment (start 85.3625 86.87) (end 87.0085 86.87) (width 0.25) (layer "F.Cu") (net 8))
 (segment (start 85.3625 85.09) (end 87.2385 85.09) (width 0.25) (layer "F.Cu") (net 9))
 (segment (start 87.2385 85.09) (end 87.3625 84.966) (width 0.25) (layer "F.Cu") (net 9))
 (segment (start 82.9575 77.3935) (end 82.9575 75.6895) (width 0.25) (layer "F.Cu") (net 6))
 (segment (start 83.105 77.3935) (end 82.9575 77.3935) (width 0.25) (layer "F.Cu") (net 6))
 (segment (start 85.3625 79.75) (end 85.3625 79.651) (width 0.25) (layer "F.Cu") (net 6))
 (segment (start 85.3625 79.651) (end 83.105 77.3935) (width 0.25) (layer "F.Cu") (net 6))
 (segment (start 96.6625 64.077487) (end 85.850487 74.8895) (width 0.25) (layer "F.Cu") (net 16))
 (segment (start 78.924 74.8895) (end 74.6625 79.151) (width 0.25) (layer "F.Cu") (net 16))
 (segment (start 85.850487 74.8895) (end 78.924 74.8895) (width 0.25) (layer "F.Cu") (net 16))
 (segment (start 96.6625 63.096116) (end 96.6625 64.077487) (width 0.25) (layer "F.Cu") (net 16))
 (segment (start 92.6625 61.98) (end 95.546384 61.98) (width 0.25) (layer "F.Cu") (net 16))
 (segment (start 95.546384 61.98) (end 96.6625 63.096116) (width 0.25) (layer "F.Cu") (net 16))
 (via (at 74.6625 79.151) (size 0.6) (drill 0.3) (layers "F.Cu" "B.Cu") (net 16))
 (via (at 92.6625 61.98) (size 0.6) (drill 0.3) (layers "F.Cu" "B.Cu") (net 16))
 (segment (start 74.6625 79.151) (end 74.6625 80.64) (width 0.25) (layer "B.Cu") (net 16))
 (segment (start 90.5675 60.505) (end 90.5125 60.56) (width 0.25) (layer "B.Cu") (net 16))
 (segment (start 91.9325 61.98) (end 92.6625 61.98) (width 0.25) (layer "B.Cu") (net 16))
 (segment (start 90.5125 60.56) (end 91.9325 61.98) (width 0.25) (layer "B.Cu") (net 16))
 (segment (start 68.6625 80.901) (end 68.6625 85.98) (width 0.25) (layer "F.Cu") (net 19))
 (segment (start 71.6625 77.901) (end 68.6625 80.901) (width 0.25) (layer "F.Cu") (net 19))
 (segment (start 68.6625 85.98) (end 70.6625 85.98) (width 0.25) (layer "F.Cu") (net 19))
 (via (at 70.6625 85.98) (size 0.6) (drill 0.3) (layers "F.Cu" "B.Cu") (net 19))
 (via (at 71.6625 77.901) (size 0.6) (drill 0.3) (layers "F.Cu" "B.Cu") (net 19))
 (segment (start 77.6625 76.98) (end 82.0125 72.48) (width 0.25) (layer "B.Cu") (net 19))
 (segment (start 82.0125 72.48) (end 89.5125 72.48) (width 0.25) (layer "B.Cu") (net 19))
 (segment (start 70.6625 85.98) (end 74.6625 85.98) (width 0.25) (layer "B.Cu") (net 19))
 (segment (start 90.5125 71.48) (end 90.5125 68.18) (width 0.25) (layer "B.Cu") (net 19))
 (segment (start 77.6625 76.98) (end 72.5835 76.98) (width 0.25) (layer "B.Cu") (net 19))
 (segment (start 89.5125 72.48) (end 90.5125 71.48) (width 0.25) (layer "B.Cu") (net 19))
 (segment (start 72.5835 76.98) (end 71.6625 77.901) (width 0.25) (layer "B.Cu") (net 19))
 (segment (start 71.6625 86.096116) (end 71.6625 88.98) (width 0.25) (layer "F.Cu") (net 18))
 (segment (start 72.6625 77.901) (end 72.6625 77.98) (width 0.25) (layer "F.Cu") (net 18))
 (segment (start 69.6625 84.096116) (end 71.6625 86.096116) (width 0.25) (layer "F.Cu") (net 18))
 (segment (start 72.6625 77.98) (end 69.6625 80.98) (width 0.25) (layer "F.Cu") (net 18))
 (segment (start 69.6625 80.98) (end 69.6625 84.096116) (width 0.25) (layer "F.Cu") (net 18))
 (via (at 71.6625 88.98) (size 0.6) (drill 0.3) (layers "F.Cu" "B.Cu") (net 18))
 (via (at 72.6625 77.901) (size 0.6) (drill 0.3) (layers "F.Cu" "B.Cu") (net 18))
 (segment (start 72.2225 89.54) (end 74.6625 89.54) (width 0.25) (layer "B.Cu") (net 18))
 (segment (start 93.0125 68.126738) (end 90.525762 65.64) (width 0.25) (layer "B.Cu") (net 18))
 (segment (start 72.8375 78.076) (end 72.6625 77.901) (width 0.25) (layer "B.Cu") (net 18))
 (segment (start 82.5125 73.48) (end 77.9165 78.076) (width 0.25) (layer "B.Cu") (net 18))
 (segment (start 74.6625 89.651) (end 74.5125 89.801) (width 0.25) (layer "B.Cu") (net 18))
 (segment (start 93.0125 70.98) (end 93.0125 68.126738) (width 0.25) (layer "B.Cu") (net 18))
 (segment (start 74.6625 89.54) (end 74.6625 89.651) (width 0.25) (layer "B.Cu") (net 18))
 (segment (start 90.525762 65.64) (end 90.5125 65.64) (width 0.25) (layer "B.Cu") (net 18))
 (segment (start 77.9165 78.076) (end 72.8375 78.076) (width 0.25) (layer "B.Cu") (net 18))
 (segment (start 82.5125 73.48) (end 90.5125 73.48) (width 0.25) (layer "B.Cu") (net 18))
 (segment (start 90.5125 73.48) (end 93.0125 70.98) (width 0.25) (layer "B.Cu") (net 18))
 (segment (start 71.6625 88.98) (end 72.2225 89.54) (width 0.25) (layer "B.Cu") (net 18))
 (segment (start 95.6625 62.98) (end 92.6625 62.98) (width 0.25) (layer "F.Cu") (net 17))
 (via (at 92.6625 62.98) (size 0.6) (drill 0.3) (layers "F.Cu" "B.Cu") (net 17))
 (via (at 95.6625 62.98) (size 0.6) (drill 0.3) (layers "F.Cu" "B.Cu") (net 17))
 (segment (start 96.6625 98.98) (end 92.1125 103.53) (width 0.25) (layer "B.Cu") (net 17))
 (segment (start 96.6625 98.98) (end 96.6625 63.98) (width 0.25) (layer "B.Cu") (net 17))
 (segment (start 92.6625 62.98) (end 90.6325 62.98) (width 0.25) (layer "B.Cu") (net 17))
 (segment (start 90.6325 62.98) (end 90.5125 63.1) (width 0.25) (layer "B.Cu") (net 17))
 (segment (start 71.5125 94.47) (end 71.5125 99.801) (width 0.25) (layer "B.Cu") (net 17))
 (segment (start 75.6625 103.78) (end 91.8625 103.78) (width 0.25) (layer "B.Cu") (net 17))
 (segment (start 96.6625 63.98) (end 95.6625 62.98) (width 0.25) (layer "B.Cu") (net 17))
 (segment (start 71.5125 99.801) (end 75.6625 103.78) (width 0.25) (layer "B.Cu") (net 17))
 (segment (start 91.8625 103.78) (end 92.1125 103.53) (width 0.25) (layer "B.Cu") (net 17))
 (segment (start 74.6625 91.32) (end 71.5125 94.47) (width 0.25) (layer "B.Cu") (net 17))
 (segment (start 72.7485 80.6985) (end 72.941 80.6985) (width 0.25) (layer "F.Cu") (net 10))
 (segment (start 72.941 80.6985) (end 74.6625 82.42) (width 0.25) (layer "F.Cu") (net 10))
 (segment (start 85.3625 90.43) (end 85.3625 92.21) (width 0.25) (layer "F.Cu") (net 22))
 (segment (start 69.6625 79.767116) (end 70.903616 78.526) (width 0.25) (layer "B.Cu") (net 23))
 (segment (start 92.7875 83.326) (end 92.7875 85.925999) (width 0.25) (layer "B.Cu") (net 23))
 (segment (start 87.9875 78.526) (end 92.7875 83.326) (width 0.25) (layer "B.Cu") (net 23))
 (segment (start 69.6625 92.48) (end 69.6625 79.767116) (width 0.25) (layer "B.Cu") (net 23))
 (segment (start 92.7875 85.925999) (end 91.6625 87.050999) (width 0.25) (layer "B.Cu") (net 23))
 (segment (start 87.9875 78.526) (end 70.903616 78.526) (width 0.25) (layer "B.Cu") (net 23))
 (segment (start 68.6625 79.33) (end 68.6625 93.98) (width 0.25) (layer "B.Cu") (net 20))
 (segment (start 75.0125 72.98) (end 68.6625 79.33) (width 0.25) (layer "B.Cu") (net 20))
 (segment (start 68.6625 93.98) (end 69.6625 94.98) (width 0.25) (layer "B.Cu") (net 20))
 (segment (start 69.5125 57.98) (end 69.5125 58.02) (width 0.25) (layer "B.Cu") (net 13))
 (segment (start 69.5125 60.56) (end 69.4325 60.48) (width 0.25) (layer "B.Cu") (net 14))
 (segment (start 69.6625 114.98) (end 70.6625 114.98) (width 0.25) (layer "F.Cu") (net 7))
 (segment (start 70.812499 115.129999) (end 73.1625 115.129999) (width 0.25) (layer "F.Cu") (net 7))
 (segment (start 70.6625 114.98) (end 70.812499 115.129999) (width 0.25) (layer "F.Cu") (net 7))
 (via (at 69.6625 114.98) (size 0.6) (drill 0.3) (layers "F.Cu" "B.Cu") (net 7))
 (segment (start 66.6625 110.88) (end 69.6625 114.98) (width 0.25) (layer "B.Cu") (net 7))
 (segment (start 68.0125 65.64) (end 66.6675 67.98) (width 0.25) (layer "B.Cu") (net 7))
 (segment (start 66.6675 67.98) (end 66.6625 110.88) (width 0.25) (layer "B.Cu") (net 7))
 (segment (start 69.5125 65.64) (end 68.0125 65.64) (width 0.25) (layer "B.Cu") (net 7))
 (segment (start 82.6625 114.98) (end 82.812499 115.129999) (width 0.25) (layer "F.Cu") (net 11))
 (segment (start 81.6625 114.98) (end 82.6625 114.98) (width 0.25) (layer "F.Cu") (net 11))
 (segment (start 82.812499 115.129999) (end 86.1625 115.129999) (width 0.25) (layer "F.Cu") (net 11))
 (via (at 81.6625 114.98) (size 0.6) (drill 0.3) (layers "F.Cu" "B.Cu") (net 11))
 (segment (start 67.6625 99.092563) (end 81.6625 114.742563) (width 0.25) (layer "B.Cu") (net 11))
 (segment (start 67.6625 72.98) (end 67.6625 99.092563) (width 0.25) (layer "B.Cu") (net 11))
 (segment (start 69.5125 68.18) (end 67.6625 72.98) (width 0.25) (layer "B.Cu") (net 11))
 (segment (start 81.6625 114.742563) (end 81.6625 114.98) (width 0.25) (layer "B.Cu") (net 11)))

